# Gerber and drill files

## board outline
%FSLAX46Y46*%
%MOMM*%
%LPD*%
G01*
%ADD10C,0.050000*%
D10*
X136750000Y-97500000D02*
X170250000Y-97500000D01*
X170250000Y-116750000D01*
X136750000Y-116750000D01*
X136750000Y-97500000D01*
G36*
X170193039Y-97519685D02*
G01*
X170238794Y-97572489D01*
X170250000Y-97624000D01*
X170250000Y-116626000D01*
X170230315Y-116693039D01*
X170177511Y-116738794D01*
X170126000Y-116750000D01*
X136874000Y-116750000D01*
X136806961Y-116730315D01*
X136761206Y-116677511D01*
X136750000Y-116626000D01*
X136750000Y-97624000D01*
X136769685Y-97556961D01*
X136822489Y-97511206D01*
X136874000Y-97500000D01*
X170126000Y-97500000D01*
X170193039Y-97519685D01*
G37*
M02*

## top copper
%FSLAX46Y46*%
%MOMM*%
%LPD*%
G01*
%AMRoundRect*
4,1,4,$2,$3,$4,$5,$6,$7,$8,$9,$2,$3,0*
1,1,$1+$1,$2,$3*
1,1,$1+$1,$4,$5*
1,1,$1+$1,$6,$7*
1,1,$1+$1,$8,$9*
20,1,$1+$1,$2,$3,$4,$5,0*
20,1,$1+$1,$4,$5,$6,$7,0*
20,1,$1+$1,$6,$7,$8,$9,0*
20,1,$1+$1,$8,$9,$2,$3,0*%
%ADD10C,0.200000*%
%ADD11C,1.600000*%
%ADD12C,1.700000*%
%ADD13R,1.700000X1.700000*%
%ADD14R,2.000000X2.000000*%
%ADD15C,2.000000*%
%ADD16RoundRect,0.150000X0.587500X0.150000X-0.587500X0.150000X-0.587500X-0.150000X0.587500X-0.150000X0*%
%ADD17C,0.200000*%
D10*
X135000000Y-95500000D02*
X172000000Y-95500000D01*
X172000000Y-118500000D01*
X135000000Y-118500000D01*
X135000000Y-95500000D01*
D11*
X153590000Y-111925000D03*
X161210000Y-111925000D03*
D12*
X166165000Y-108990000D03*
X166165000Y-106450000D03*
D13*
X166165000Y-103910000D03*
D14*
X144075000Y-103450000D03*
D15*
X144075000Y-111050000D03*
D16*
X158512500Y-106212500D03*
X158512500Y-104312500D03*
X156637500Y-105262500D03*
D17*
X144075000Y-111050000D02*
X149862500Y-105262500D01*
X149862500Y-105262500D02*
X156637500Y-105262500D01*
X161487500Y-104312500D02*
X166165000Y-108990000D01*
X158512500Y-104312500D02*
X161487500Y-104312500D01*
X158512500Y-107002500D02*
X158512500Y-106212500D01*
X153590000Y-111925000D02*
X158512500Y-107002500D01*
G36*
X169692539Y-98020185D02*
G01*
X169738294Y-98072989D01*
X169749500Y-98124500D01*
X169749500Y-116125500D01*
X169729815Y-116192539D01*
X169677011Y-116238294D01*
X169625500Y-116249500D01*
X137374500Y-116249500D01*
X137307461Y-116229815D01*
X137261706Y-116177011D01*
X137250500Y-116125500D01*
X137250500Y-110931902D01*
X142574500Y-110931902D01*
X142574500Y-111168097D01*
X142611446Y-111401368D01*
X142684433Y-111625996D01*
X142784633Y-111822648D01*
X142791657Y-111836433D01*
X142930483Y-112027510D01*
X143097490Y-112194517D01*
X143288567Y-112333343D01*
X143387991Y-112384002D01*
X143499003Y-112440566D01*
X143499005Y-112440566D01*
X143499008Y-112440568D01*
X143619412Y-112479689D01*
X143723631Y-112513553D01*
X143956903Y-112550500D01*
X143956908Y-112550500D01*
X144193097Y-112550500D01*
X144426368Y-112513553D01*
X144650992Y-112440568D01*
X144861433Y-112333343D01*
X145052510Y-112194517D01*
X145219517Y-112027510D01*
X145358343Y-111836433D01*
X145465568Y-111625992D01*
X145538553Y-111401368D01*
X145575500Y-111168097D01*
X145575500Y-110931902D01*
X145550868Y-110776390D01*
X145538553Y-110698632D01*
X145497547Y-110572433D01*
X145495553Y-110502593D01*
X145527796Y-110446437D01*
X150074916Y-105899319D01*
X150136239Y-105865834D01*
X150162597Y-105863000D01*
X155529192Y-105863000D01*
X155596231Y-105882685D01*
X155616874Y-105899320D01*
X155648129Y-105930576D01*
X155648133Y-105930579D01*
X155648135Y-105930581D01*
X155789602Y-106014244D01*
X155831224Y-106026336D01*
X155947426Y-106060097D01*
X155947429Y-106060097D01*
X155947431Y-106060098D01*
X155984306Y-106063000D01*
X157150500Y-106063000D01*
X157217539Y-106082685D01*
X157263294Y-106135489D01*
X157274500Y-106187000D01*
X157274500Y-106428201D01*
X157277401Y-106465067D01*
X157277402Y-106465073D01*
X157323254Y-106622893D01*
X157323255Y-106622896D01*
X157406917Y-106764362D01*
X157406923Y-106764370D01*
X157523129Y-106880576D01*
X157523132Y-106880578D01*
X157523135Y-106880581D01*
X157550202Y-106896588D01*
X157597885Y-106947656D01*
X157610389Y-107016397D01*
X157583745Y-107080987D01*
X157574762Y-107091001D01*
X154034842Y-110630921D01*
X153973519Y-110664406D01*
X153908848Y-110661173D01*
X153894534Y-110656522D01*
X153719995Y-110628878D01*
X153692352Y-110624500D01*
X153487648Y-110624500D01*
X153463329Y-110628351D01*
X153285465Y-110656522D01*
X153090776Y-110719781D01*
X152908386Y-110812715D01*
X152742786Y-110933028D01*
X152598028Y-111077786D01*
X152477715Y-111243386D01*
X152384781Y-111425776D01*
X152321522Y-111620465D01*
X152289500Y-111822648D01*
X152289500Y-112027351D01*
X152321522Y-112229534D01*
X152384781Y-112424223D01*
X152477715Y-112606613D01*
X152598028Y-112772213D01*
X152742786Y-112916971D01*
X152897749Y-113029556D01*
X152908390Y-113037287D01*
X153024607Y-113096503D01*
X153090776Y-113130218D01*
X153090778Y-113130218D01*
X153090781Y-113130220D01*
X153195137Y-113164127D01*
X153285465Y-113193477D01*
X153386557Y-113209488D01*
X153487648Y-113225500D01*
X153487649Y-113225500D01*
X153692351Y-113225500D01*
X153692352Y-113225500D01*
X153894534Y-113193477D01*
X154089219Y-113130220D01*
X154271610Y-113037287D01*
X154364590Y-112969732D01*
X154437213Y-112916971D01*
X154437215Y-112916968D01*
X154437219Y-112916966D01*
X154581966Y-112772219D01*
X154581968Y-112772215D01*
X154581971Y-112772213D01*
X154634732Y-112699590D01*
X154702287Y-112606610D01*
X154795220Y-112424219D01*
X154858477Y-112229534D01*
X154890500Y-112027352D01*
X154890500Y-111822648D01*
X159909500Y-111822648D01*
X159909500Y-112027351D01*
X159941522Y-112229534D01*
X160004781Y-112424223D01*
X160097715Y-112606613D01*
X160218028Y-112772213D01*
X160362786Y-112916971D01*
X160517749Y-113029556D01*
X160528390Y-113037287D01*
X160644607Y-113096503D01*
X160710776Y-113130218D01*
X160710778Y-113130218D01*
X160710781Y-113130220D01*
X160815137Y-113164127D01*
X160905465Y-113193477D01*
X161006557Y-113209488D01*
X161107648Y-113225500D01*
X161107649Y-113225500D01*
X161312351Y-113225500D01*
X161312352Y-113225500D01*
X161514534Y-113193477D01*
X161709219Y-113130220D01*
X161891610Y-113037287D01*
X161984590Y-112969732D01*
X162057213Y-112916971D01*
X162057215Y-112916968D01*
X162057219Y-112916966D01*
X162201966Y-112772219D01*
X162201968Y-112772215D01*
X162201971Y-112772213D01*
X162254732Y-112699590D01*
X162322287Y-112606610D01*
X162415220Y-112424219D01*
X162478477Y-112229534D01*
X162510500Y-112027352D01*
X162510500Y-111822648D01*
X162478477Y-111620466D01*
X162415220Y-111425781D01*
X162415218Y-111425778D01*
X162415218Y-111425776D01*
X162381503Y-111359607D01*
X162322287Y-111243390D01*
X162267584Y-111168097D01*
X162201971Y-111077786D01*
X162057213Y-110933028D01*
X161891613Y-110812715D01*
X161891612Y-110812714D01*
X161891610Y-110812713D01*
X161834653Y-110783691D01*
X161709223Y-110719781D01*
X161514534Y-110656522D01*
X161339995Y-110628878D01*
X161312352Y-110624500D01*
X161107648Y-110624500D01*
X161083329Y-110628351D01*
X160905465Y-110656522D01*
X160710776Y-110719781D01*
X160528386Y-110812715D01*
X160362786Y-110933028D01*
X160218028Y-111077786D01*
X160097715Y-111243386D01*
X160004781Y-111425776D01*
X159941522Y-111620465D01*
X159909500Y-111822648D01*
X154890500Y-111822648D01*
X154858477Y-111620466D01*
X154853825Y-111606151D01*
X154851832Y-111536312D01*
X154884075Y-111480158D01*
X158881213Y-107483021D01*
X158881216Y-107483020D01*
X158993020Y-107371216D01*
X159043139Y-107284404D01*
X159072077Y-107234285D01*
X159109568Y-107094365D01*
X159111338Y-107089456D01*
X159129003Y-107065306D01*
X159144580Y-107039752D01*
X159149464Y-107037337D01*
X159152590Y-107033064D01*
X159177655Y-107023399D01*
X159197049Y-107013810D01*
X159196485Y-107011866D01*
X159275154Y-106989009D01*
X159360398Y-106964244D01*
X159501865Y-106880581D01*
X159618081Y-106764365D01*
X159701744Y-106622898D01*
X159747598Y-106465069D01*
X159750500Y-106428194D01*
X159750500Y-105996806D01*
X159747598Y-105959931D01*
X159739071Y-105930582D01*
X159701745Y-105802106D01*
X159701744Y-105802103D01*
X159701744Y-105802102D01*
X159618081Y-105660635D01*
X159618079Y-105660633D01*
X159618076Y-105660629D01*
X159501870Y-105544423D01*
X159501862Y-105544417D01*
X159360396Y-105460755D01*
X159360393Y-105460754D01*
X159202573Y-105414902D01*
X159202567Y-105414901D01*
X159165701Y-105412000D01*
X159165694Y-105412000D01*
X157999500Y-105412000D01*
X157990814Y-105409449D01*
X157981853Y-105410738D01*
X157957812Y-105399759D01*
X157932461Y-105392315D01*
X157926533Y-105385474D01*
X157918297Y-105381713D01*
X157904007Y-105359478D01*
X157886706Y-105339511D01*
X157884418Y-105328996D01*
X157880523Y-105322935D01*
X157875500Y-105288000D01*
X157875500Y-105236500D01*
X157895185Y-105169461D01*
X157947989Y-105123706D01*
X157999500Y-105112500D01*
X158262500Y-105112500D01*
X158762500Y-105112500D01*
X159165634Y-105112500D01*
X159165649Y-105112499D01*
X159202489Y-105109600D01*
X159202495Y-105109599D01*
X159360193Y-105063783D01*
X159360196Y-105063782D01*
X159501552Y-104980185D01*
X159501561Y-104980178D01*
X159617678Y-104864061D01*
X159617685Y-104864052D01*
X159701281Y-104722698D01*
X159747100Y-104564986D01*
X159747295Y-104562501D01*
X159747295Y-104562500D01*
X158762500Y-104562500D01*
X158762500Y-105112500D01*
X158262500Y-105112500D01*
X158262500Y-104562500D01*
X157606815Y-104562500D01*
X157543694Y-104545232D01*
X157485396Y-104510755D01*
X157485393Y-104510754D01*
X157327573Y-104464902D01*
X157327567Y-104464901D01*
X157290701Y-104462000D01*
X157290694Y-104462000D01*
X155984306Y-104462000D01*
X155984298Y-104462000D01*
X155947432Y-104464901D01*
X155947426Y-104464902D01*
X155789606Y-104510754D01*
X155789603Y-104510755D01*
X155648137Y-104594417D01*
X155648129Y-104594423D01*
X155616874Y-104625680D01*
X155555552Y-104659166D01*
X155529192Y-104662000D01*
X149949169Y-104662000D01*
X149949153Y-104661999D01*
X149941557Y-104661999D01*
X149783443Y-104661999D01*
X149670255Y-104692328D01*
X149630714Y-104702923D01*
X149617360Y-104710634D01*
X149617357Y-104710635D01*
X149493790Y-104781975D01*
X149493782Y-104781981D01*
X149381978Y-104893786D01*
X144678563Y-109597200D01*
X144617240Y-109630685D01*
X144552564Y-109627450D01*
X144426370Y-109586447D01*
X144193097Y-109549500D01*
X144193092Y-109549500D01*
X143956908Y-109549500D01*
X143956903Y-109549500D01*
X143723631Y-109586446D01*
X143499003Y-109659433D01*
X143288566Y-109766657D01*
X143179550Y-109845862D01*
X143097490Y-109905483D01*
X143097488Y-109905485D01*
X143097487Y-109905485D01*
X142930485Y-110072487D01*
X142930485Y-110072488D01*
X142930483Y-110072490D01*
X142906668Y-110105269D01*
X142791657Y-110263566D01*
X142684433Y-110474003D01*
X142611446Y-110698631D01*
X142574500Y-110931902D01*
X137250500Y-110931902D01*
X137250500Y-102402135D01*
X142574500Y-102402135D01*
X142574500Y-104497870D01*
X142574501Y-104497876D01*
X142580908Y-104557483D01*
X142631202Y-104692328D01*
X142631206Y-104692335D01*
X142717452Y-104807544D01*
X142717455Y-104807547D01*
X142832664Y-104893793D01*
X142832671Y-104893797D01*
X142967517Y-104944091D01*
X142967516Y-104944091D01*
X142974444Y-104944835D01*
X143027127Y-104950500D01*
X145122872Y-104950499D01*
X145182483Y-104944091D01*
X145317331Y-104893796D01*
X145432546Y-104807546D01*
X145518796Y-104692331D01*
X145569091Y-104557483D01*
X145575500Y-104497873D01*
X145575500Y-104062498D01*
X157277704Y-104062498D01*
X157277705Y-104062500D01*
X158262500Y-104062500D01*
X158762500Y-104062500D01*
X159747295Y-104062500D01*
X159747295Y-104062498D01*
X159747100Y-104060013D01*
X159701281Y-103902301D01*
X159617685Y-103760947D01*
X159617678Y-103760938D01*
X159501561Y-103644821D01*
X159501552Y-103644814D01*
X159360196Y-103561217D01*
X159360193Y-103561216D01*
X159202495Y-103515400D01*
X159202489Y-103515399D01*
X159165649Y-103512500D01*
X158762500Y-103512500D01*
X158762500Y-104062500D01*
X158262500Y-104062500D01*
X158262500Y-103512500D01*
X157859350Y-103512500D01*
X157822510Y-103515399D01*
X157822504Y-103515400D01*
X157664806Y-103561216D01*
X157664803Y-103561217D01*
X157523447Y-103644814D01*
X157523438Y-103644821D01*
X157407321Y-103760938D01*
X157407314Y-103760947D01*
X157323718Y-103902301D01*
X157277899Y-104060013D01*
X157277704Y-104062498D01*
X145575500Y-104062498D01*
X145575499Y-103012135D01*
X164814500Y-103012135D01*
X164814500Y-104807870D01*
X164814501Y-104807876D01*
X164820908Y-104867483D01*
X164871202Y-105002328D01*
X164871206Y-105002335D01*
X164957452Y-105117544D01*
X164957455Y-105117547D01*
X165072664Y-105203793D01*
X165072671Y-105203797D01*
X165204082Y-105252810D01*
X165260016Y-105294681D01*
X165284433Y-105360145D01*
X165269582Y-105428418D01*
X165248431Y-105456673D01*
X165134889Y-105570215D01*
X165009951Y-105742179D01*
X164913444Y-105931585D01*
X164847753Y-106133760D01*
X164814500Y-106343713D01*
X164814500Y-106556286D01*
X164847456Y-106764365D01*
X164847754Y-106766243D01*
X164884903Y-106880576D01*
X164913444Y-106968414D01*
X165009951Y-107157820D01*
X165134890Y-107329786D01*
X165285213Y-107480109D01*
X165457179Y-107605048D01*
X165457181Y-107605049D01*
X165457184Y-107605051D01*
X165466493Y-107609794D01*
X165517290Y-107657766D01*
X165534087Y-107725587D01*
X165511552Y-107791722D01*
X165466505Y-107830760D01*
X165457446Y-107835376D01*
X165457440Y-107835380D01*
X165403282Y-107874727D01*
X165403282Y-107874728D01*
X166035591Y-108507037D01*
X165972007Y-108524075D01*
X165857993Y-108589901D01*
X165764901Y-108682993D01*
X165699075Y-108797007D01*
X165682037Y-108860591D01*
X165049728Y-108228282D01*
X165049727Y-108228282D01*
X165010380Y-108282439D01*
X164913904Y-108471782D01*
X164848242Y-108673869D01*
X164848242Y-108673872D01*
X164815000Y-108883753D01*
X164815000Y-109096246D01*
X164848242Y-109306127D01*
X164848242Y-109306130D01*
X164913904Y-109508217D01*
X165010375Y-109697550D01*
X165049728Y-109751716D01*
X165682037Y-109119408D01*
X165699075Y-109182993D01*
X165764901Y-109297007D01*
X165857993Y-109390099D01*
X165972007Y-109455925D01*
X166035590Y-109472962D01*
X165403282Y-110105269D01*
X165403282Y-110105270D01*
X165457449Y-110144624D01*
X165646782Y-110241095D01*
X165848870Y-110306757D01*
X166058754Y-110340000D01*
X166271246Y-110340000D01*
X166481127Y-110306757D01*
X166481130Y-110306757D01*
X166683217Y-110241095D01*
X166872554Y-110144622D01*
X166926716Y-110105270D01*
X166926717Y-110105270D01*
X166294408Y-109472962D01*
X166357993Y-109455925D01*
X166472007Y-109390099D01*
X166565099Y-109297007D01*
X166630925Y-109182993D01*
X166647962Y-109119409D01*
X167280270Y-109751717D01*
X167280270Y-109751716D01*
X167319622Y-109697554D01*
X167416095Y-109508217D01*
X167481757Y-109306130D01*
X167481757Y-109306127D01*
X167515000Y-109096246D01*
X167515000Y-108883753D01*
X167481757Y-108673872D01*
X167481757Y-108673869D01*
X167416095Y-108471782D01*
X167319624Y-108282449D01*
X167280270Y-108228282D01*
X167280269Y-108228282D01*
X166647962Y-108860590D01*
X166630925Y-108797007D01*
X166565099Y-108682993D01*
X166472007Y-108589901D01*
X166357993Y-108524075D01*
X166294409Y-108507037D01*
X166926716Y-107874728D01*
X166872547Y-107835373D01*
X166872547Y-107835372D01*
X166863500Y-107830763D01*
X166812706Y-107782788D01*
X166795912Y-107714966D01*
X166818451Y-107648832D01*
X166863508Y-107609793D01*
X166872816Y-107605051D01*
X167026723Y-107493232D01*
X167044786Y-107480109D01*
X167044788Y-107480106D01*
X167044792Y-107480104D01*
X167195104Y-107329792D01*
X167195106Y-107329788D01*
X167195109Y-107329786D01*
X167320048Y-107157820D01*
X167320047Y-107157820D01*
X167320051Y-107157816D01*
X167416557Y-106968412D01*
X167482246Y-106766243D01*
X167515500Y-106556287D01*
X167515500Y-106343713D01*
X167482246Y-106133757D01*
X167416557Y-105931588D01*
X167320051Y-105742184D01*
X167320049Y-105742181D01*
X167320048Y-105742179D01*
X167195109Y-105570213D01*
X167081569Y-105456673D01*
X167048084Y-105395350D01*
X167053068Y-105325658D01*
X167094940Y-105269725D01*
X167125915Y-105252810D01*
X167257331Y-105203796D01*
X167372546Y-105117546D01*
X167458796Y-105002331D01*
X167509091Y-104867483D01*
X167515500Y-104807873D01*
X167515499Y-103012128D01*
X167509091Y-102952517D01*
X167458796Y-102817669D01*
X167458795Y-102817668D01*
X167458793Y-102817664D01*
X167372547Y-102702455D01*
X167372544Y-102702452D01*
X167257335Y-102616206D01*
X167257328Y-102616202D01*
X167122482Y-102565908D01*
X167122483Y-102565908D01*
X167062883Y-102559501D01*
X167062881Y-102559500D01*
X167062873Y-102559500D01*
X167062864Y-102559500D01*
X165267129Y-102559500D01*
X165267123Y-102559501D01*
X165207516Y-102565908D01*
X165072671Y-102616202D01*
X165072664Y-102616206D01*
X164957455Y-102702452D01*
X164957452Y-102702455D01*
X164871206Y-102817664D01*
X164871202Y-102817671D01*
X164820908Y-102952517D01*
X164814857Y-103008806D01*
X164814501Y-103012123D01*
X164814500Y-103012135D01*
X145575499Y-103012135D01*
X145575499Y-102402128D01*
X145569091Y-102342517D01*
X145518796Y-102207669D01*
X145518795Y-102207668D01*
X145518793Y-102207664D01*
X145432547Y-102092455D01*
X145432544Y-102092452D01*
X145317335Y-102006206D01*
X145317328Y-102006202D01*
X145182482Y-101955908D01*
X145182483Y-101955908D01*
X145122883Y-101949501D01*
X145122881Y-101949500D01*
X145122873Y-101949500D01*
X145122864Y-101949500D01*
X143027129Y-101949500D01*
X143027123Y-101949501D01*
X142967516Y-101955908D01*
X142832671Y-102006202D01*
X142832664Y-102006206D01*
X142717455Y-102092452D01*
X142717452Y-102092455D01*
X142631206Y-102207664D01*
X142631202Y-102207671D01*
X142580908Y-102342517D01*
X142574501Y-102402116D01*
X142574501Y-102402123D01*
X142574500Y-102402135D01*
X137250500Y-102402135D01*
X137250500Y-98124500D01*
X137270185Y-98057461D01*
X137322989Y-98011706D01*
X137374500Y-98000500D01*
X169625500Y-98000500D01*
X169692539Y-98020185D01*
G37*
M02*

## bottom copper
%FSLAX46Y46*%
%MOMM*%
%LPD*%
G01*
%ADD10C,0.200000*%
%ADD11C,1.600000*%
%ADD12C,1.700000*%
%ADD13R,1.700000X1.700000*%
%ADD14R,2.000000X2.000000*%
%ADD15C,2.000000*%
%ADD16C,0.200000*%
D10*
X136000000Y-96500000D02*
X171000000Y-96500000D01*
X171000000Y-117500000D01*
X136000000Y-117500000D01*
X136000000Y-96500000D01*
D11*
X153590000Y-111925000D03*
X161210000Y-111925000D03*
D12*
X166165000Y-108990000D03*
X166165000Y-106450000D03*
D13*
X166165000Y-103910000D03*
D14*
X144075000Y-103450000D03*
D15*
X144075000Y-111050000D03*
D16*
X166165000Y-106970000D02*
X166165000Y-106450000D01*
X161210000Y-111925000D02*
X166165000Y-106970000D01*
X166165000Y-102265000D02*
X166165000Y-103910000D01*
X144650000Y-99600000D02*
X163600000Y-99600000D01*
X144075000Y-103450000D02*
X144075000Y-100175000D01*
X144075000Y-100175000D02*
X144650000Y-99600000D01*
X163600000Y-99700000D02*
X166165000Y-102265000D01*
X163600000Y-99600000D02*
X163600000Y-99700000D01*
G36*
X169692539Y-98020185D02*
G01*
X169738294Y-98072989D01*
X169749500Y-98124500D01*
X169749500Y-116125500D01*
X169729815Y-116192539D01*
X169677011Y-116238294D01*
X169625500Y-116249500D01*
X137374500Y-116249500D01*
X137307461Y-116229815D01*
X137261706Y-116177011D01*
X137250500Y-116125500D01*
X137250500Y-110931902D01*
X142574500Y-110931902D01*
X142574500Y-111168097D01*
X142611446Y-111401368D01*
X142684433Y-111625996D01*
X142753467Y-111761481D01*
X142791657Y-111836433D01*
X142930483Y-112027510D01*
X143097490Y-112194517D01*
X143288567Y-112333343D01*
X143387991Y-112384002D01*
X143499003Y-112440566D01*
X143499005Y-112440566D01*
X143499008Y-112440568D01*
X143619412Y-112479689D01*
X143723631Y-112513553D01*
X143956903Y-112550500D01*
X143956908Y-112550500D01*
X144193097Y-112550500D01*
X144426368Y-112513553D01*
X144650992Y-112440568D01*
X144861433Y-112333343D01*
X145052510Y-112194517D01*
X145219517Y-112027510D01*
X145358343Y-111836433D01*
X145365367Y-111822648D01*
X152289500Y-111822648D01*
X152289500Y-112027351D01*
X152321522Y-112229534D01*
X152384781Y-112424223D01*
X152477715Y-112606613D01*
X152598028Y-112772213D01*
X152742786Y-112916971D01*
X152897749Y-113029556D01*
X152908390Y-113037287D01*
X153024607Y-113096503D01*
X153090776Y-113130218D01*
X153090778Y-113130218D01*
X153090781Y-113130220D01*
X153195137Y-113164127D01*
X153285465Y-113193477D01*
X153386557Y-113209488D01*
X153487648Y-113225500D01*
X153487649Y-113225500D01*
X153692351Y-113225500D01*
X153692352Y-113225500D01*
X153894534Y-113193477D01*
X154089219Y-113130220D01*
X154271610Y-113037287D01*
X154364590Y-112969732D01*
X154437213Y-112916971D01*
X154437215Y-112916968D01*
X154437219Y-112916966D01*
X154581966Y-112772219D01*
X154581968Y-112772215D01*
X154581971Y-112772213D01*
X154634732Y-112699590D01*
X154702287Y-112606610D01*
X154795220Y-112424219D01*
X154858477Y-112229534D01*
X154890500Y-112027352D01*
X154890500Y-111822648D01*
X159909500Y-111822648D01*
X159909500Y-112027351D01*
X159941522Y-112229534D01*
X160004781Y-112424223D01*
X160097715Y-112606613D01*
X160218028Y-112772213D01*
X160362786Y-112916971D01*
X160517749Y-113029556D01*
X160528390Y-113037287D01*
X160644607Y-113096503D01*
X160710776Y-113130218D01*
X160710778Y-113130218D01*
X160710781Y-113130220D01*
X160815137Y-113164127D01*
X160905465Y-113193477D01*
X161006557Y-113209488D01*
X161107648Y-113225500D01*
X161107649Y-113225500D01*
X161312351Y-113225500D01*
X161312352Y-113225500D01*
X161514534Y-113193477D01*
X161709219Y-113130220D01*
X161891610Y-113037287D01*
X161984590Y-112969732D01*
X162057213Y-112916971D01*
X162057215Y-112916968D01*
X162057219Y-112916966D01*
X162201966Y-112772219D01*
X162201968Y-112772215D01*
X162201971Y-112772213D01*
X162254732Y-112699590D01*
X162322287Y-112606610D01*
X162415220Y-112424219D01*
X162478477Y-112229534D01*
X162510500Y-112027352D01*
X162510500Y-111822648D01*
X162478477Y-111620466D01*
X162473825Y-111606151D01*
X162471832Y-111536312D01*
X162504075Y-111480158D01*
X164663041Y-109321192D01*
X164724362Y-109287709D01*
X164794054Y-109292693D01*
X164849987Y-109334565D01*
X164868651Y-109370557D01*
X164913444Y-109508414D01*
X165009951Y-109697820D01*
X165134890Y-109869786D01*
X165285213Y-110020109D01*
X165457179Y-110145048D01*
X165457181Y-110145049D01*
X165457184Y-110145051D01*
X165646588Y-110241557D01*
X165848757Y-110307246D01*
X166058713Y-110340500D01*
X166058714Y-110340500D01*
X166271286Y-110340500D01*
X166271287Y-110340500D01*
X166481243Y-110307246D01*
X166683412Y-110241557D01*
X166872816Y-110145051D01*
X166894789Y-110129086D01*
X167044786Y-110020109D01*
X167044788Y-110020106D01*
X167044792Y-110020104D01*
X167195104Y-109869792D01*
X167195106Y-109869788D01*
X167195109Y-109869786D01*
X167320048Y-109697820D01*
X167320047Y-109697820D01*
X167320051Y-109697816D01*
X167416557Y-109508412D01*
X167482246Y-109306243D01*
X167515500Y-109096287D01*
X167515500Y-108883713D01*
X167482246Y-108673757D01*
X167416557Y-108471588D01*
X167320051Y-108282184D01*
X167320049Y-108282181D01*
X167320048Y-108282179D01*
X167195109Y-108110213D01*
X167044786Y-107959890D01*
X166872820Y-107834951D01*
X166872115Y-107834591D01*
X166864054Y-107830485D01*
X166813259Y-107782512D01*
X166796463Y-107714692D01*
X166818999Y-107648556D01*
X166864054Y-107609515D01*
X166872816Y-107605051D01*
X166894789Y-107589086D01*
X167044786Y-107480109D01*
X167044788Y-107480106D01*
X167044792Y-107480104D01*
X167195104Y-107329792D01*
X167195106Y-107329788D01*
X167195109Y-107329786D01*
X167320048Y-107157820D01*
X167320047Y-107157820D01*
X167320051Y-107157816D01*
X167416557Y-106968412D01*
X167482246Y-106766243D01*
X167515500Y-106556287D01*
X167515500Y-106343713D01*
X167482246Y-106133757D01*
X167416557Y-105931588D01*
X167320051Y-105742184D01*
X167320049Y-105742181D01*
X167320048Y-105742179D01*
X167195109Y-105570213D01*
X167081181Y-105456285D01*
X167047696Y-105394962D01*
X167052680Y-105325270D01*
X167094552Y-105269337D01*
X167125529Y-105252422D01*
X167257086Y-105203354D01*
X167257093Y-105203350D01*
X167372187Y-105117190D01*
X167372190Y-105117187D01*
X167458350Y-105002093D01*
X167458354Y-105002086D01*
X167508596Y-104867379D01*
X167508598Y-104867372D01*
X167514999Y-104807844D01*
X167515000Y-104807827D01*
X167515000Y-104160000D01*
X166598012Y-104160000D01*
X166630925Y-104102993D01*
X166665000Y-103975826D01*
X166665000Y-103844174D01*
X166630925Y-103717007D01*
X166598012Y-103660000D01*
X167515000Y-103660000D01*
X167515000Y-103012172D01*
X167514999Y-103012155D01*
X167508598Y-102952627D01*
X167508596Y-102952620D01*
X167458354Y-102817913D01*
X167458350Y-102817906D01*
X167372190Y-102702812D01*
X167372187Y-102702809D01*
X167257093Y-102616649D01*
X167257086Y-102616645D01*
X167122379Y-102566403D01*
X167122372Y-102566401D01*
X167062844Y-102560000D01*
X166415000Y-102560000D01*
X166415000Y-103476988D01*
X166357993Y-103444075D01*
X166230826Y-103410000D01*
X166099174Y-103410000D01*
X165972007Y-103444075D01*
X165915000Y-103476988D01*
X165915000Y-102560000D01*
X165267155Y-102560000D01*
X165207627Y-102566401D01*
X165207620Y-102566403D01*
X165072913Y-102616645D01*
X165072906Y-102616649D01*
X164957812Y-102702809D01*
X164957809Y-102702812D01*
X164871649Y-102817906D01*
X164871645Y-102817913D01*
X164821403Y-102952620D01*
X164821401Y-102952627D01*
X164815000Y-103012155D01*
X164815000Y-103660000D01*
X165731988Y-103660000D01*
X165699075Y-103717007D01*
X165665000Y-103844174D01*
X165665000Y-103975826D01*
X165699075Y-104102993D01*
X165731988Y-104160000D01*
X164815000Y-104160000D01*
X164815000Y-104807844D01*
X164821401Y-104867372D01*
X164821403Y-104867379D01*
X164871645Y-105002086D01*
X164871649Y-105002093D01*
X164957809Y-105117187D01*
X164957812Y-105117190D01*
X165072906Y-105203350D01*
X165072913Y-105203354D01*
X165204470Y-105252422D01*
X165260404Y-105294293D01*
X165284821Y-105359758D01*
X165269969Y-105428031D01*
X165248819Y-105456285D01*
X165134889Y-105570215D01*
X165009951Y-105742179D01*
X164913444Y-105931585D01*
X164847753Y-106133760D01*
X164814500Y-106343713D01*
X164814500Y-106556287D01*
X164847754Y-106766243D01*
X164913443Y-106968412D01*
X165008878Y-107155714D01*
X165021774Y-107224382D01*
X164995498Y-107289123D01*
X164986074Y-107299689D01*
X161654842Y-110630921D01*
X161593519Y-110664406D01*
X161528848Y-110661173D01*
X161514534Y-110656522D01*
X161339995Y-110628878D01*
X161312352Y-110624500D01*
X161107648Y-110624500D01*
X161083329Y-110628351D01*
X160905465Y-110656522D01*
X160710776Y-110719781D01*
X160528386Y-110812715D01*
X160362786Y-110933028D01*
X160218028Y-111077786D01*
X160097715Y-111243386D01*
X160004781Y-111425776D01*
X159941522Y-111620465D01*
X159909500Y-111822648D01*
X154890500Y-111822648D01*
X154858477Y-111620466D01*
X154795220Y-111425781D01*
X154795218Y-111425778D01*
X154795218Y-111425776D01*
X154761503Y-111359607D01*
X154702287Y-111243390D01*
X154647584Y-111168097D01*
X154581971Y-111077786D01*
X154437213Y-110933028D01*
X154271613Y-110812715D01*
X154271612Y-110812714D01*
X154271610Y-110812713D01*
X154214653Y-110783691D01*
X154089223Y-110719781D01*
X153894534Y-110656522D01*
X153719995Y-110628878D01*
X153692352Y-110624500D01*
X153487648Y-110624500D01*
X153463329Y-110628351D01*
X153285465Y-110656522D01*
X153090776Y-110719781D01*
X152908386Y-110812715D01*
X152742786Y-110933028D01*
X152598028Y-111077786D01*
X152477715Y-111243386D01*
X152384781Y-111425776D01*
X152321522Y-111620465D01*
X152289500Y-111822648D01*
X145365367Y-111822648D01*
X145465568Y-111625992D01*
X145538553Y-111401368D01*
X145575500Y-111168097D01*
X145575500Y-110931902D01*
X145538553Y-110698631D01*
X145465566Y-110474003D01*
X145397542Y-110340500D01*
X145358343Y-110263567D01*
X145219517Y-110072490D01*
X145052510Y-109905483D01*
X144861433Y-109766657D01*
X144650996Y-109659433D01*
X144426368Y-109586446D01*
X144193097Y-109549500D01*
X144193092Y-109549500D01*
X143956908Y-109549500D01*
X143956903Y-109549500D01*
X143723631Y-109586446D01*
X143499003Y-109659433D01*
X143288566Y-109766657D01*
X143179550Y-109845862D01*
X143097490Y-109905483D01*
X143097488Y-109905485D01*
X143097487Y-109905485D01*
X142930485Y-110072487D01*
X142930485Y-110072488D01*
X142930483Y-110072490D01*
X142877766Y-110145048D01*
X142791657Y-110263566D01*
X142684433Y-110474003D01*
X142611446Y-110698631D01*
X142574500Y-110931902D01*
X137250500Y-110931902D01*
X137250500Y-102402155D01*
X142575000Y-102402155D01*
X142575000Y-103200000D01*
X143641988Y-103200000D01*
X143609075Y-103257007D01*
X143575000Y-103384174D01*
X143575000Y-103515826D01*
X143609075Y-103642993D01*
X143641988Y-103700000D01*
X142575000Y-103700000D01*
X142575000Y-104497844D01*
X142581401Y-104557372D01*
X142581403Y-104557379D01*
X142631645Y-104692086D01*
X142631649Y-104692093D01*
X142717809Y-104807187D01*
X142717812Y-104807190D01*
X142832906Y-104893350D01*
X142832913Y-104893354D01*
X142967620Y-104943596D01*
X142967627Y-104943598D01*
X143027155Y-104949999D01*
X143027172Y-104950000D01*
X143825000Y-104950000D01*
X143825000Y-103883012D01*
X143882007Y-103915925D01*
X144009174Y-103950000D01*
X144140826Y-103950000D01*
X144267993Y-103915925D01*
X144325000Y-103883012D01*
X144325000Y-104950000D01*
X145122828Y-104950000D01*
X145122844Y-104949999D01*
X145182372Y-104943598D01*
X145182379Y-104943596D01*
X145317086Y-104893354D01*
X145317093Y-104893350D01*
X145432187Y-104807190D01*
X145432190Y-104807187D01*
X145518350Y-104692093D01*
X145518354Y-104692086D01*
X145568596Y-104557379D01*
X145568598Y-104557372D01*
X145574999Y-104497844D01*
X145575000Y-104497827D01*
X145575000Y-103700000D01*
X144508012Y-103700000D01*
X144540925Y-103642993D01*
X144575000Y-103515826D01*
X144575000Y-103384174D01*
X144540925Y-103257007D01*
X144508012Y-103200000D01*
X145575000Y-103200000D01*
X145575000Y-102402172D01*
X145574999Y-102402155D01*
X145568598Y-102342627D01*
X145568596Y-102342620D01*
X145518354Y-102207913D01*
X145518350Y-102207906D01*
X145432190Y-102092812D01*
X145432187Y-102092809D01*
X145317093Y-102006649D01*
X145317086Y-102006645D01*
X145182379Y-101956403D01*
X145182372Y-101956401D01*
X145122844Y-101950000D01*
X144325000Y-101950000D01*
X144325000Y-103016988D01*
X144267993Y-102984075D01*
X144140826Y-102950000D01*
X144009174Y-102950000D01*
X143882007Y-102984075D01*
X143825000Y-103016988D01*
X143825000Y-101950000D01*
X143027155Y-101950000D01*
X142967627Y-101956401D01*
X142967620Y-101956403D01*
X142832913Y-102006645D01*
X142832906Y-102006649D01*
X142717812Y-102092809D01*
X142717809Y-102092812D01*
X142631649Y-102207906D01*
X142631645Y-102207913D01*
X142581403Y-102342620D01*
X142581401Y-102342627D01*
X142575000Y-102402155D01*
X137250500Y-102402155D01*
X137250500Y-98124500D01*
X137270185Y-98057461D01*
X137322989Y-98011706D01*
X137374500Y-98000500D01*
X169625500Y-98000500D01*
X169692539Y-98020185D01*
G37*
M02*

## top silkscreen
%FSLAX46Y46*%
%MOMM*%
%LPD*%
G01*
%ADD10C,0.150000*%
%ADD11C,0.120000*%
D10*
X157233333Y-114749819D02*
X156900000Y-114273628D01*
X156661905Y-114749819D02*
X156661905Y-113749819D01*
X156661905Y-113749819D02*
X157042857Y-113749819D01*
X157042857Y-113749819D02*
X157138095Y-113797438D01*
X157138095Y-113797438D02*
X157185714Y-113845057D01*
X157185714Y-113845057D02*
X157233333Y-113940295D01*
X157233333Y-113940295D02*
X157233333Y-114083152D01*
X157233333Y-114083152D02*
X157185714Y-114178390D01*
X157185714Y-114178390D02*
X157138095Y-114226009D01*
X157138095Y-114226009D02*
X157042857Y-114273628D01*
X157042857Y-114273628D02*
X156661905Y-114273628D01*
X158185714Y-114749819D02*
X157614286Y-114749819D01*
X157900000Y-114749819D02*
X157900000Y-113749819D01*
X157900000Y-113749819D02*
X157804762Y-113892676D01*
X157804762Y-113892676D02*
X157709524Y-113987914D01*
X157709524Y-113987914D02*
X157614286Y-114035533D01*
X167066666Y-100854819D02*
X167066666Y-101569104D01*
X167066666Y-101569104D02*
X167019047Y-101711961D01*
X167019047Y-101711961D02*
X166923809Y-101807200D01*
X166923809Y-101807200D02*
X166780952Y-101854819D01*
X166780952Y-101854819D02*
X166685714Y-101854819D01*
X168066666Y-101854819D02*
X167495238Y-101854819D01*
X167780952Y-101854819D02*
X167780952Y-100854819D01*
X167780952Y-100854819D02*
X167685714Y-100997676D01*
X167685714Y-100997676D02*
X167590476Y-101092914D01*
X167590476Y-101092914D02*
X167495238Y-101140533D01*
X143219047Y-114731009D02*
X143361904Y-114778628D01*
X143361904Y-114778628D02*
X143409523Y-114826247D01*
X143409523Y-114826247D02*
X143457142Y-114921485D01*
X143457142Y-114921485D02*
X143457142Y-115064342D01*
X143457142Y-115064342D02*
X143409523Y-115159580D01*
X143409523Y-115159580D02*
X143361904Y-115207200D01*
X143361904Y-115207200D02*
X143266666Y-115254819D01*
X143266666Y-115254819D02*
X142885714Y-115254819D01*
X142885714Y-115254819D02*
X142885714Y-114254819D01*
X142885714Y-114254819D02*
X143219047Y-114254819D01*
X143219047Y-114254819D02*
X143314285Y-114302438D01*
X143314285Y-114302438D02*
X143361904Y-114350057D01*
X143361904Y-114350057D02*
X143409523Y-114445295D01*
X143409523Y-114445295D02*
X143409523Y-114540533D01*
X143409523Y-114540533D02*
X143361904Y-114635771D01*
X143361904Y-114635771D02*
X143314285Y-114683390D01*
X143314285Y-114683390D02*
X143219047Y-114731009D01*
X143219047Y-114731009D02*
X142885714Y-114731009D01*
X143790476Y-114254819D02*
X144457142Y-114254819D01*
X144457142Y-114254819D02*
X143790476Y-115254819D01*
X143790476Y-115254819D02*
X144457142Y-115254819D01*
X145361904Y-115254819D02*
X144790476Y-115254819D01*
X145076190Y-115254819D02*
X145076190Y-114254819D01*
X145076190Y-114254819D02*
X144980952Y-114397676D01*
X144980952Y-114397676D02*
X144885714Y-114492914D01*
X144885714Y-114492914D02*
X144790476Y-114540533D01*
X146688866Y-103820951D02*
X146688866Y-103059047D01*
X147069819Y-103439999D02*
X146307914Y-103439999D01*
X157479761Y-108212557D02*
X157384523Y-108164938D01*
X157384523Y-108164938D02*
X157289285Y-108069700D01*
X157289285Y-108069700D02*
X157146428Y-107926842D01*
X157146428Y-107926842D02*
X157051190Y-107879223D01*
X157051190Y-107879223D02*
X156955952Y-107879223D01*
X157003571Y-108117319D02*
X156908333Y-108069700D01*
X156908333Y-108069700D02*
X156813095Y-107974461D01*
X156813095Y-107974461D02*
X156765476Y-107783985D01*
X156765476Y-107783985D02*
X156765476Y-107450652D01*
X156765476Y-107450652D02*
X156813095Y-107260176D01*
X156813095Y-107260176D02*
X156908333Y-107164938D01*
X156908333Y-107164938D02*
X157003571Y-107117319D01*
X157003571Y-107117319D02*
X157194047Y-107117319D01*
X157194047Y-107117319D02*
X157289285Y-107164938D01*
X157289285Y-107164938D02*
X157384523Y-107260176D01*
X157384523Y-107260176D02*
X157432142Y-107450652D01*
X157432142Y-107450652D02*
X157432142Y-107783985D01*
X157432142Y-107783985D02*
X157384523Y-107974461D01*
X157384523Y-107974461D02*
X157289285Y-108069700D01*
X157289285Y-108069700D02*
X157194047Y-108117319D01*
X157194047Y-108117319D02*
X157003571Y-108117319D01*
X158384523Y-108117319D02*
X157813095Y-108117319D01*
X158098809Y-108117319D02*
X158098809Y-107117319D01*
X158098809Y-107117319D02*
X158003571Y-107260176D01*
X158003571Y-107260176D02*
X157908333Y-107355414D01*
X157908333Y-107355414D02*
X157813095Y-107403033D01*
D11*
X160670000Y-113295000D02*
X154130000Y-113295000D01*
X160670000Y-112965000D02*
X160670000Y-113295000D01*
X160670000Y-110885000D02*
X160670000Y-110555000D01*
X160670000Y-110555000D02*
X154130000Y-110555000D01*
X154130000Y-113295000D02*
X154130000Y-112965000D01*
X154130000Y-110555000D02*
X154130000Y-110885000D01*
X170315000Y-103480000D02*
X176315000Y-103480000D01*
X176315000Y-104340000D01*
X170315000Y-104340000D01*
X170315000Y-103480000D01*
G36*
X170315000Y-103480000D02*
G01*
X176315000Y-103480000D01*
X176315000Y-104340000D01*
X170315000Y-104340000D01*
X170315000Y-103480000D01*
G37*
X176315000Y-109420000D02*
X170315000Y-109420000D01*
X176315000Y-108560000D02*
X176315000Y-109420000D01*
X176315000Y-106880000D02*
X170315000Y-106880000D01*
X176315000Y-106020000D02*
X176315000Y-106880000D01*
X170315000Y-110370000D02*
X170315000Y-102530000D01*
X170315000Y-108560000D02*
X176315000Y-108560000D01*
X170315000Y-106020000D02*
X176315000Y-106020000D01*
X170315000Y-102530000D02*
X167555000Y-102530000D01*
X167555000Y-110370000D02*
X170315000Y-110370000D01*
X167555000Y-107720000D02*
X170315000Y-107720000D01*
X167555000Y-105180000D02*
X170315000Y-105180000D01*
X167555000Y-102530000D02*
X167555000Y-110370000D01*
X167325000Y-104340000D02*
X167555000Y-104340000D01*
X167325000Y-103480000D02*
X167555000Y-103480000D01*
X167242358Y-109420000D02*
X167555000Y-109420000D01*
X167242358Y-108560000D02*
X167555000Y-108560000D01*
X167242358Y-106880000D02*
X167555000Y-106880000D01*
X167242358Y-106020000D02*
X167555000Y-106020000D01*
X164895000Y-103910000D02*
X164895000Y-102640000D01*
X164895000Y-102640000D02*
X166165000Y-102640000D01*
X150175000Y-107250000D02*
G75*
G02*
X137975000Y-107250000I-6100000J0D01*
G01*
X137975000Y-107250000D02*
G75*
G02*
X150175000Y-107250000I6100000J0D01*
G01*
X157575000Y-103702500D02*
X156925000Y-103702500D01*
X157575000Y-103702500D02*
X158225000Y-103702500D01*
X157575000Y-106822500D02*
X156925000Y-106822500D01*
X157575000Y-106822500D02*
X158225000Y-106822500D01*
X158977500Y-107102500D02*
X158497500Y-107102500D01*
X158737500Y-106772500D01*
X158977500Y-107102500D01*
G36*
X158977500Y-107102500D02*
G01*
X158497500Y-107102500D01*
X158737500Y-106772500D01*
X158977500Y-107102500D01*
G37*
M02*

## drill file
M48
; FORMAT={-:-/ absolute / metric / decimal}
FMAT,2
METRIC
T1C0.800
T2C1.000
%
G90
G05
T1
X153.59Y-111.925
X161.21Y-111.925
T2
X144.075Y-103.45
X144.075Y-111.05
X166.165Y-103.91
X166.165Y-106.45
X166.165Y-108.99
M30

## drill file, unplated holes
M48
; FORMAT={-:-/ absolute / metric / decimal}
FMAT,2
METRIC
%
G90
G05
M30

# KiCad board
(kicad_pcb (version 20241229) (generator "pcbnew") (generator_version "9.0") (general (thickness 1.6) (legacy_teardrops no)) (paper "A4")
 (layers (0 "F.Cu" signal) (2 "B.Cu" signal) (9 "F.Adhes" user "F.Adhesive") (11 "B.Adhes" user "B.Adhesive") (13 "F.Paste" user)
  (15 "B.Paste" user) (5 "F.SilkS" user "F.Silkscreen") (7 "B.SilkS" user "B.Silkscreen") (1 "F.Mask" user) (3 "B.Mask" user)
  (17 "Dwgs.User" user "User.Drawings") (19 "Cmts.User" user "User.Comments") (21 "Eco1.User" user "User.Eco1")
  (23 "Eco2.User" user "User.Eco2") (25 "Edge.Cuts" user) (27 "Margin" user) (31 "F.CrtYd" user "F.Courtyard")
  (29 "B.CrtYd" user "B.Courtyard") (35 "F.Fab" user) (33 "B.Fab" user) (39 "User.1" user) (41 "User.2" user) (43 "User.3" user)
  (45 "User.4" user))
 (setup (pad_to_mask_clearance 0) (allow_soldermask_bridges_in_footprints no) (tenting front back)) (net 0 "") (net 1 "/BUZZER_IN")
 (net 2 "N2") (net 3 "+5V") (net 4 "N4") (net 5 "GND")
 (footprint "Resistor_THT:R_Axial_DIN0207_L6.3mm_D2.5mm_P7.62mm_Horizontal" (layer "F.Cu") (at 161.21 111.925 180)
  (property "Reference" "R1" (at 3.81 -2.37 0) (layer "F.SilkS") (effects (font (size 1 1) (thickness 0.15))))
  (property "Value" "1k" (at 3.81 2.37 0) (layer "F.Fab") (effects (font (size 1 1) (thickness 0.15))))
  (fp_line (start 7.08 1.37) (end 7.08 1.04) (stroke (width 0.12) (type solid)) (layer "F.SilkS"))
  (fp_line (start 7.08 -1.37) (end 7.08 -1.04) (stroke (width 0.12) (type solid)) (layer "F.SilkS"))
  (fp_line (start 0.54 1.37) (end 7.08 1.37) (stroke (width 0.12) (type solid)) (layer "F.SilkS"))
  (fp_line (start 0.54 1.04) (end 0.54 1.37) (stroke (width 0.12) (type solid)) (layer "F.SilkS"))
  (fp_line (start 0.54 -1.04) (end 0.54 -1.37) (stroke (width 0.12) (type solid)) (layer "F.SilkS"))
  (fp_line (start 0.54 -1.37) (end 7.08 -1.37) (stroke (width 0.12) (type solid)) (layer "F.SilkS"))
  (pad "1" thru_hole circle (at 0 0 180) (size 1.6 1.6) (drill 0.8) (layers "*.Cu" "*.Mask") (remove_unused_layers no) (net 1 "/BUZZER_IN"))
  (pad "2" thru_hole circle (at 7.62 0 180) (size 1.6 1.6) (drill 0.8) (layers "*.Cu" "*.Mask") (remove_unused_layers no) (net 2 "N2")))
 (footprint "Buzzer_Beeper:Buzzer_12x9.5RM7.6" (layer "F.Cu") (at 144.075 103.45 -90)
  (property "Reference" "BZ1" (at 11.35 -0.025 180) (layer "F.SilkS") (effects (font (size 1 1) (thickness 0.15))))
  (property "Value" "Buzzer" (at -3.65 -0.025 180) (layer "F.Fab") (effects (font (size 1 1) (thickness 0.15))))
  (fp_circle (center 3.8 0) (end 9.9 0) (stroke (width 0.12) (type solid)) (fill no) (layer "F.SilkS"))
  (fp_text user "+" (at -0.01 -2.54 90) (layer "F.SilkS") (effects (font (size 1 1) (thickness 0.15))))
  (pad "1" thru_hole rect (at 0 0 270) (size 2 2) (drill 1) (layers "*.Cu" "*.Mask") (remove_unused_layers no) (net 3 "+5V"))
  (pad "2" thru_hole circle (at 7.6 0 270) (size 2 2) (drill 1) (layers "*.Cu" "*.Mask") (remove_unused_layers no) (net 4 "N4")))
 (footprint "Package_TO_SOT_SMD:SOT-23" (layer "F.Cu") (at 157.575 105.2625 180)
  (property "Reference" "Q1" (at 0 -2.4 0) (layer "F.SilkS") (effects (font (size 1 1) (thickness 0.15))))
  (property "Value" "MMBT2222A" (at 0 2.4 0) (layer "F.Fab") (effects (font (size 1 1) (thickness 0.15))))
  (fp_line (start 0 1.56) (end 0.65 1.56) (stroke (width 0.12) (type solid)) (layer "F.SilkS"))
  (fp_line (start 0 1.56) (end -0.65 1.56) (stroke (width 0.12) (type solid)) (layer "F.SilkS"))
  (fp_line (start 0 -1.56) (end 0.65 -1.56) (stroke (width 0.12) (type solid)) (layer "F.SilkS"))
  (fp_line (start 0 -1.56) (end -0.65 -1.56) (stroke (width 0.12) (type solid)) (layer "F.SilkS"))
  (fp_poly (pts (xy -1.1625 -1.51) (xy -1.4025 -1.84) (xy -0.9225 -1.84)) (stroke (width 0.12) (type solid)) (fill yes) (layer "F.SilkS"))
  (pad "1" smd roundrect (at -0.9375 -0.95 180) (size 1.475 0.6) (layers "F.Cu" "F.Mask" "F.Paste") (roundrect_rratio 0.25) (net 2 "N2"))
  (pad "2" smd roundrect (at -0.9375 0.95 180) (size 1.475 0.6) (layers "F.Cu" "F.Mask" "F.Paste") (roundrect_rratio 0.25) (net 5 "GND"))
  (pad "3" smd roundrect (at 0.9375 0 180) (size 1.475 0.6) (layers "F.Cu" "F.Mask" "F.Paste") (roundrect_rratio 0.25) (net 4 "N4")))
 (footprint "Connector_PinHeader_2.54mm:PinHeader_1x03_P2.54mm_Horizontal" (layer "F.Cu") (at 166.165 103.91)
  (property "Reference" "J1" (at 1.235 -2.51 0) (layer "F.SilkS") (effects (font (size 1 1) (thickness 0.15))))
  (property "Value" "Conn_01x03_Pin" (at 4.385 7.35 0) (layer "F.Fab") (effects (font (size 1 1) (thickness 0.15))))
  (fp_line (start -1.27 -1.27) (end 0 -1.27) (stroke (width 0.12) (type solid)) (layer "F.SilkS"))
  (fp_line (start -1.27 0) (end -1.27 -1.27) (stroke (width 0.12) (type solid)) (layer "F.SilkS"))
  (fp_line (start 1.077358 2.11) (end 1.39 2.11) (stroke (width 0.12) (type solid)) (layer "F.SilkS"))
  (fp_line (start 1.077358 2.97) (end 1.39 2.97) (stroke (width 0.12) (type solid)) (layer "F.SilkS"))
  (fp_line (start 1.077358 4.65) (end 1.39 4.65) (stroke (width 0.12) (type solid)) (layer "F.SilkS"))
  (fp_line (start 1.077358 5.51) (end 1.39 5.51) (stroke (width 0.12) (type solid)) (layer "F.SilkS"))
  (fp_line (start 1.16 -0.43) (end 1.39 -0.43) (stroke (width 0.12) (type solid)) (layer "F.SilkS"))
  (fp_line (start 1.16 0.43) (end 1.39 0.43) (stroke (width 0.12) (type solid)) (layer "F.SilkS"))
  (fp_line (start 1.39 -1.38) (end 1.39 6.46) (stroke (width 0.12) (type solid)) (layer "F.SilkS"))
  (fp_line (start 1.39 1.27) (end 4.15 1.27) (stroke (width 0.12) (type solid)) (layer "F.SilkS"))
  (fp_line (start 1.39 3.81) (end 4.15 3.81) (stroke (width 0.12) (type solid)) (layer "F.SilkS"))
  (fp_line (start 1.39 6.46) (end 4.15 6.46) (stroke (width 0.12) (type solid)) (layer "F.SilkS"))
  (fp_line (start 4.15 -1.38) (end 1.39 -1.38) (stroke (width 0.12) (type solid)) (layer "F.SilkS"))
  (fp_line (start 4.15 2.11) (end 10.15 2.11) (stroke (width 0.12) (type solid)) (layer "F.SilkS"))
  (fp_line (start 4.15 4.65) (end 10.15 4.65) (stroke (width 0.12) (type solid)) (layer "F.SilkS"))
  (fp_line (start 4.15 6.46) (end 4.15 -1.38) (stroke (width 0.12) (type solid)) (layer "F.SilkS"))
  (fp_line (start 10.15 2.11) (end 10.15 2.97) (stroke (width 0.12) (type solid)) (layer "F.SilkS"))
  (fp_line (start 10.15 2.97) (end 4.15 2.97) (stroke (width 0.12) (type solid)) (layer "F.SilkS"))
  (fp_line (start 10.15 4.65) (end 10.15 5.51) (stroke (width 0.12) (type solid)) (layer "F.SilkS"))
  (fp_line (start 10.15 5.51) (end 4.15 5.51) (stroke (width 0.12) (type solid)) (layer "F.SilkS"))
  (fp_rect (start 4.15 -0.43) (end 10.15 0.43) (stroke (width 0.12) (type solid)) (fill yes) (layer "F.SilkS"))
  (pad "1" thru_hole rect (at 0 0) (size 1.7 1.7) (drill 1) (layers "*.Cu" "*.Mask") (remove_unused_layers no) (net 3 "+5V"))
  (pad "2" thru_hole circle (at 0 2.54) (size 1.7 1.7) (drill 1) (layers "*.Cu" "*.Mask") (remove_unused_layers no) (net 1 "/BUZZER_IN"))
  (pad "3" thru_hole circle (at 0 5.08) (size 1.7 1.7) (drill 1) (layers "*.Cu" "*.Mask") (remove_unused_layers no) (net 5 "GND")))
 (gr_rect (start 135 95.5) (end 172 118.5) (stroke (width 0.2) (type default)) (fill no) (layer "F.Cu"))
 (gr_rect (start 136 96.5) (end 171 117.5) (stroke (width 0.2) (type default)) (fill no) (layer "B.Cu"))
 (gr_rect (start 136.75 97.5) (end 170.25 116.75) (stroke (width 0.05) (type default)) (fill no) (layer "Edge.Cuts"))
 (segment (start 166.165 102.265) (end 166.165 103.91) (width 0.2) (layer "B.Cu") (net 3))
 (segment (start 144.65 99.6) (end 163.6 99.6) (width 0.2) (layer "B.Cu") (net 3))
 (segment (start 144.075 103.45) (end 144.075 100.175) (width 0.2) (layer "B.Cu") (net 3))
 (segment (start 144.075 100.175) (end 144.65 99.6) (width 0.2) (layer "B.Cu") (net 3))
 (segment (start 163.6 99.7) (end 166.165 102.265) (width 0.2) (layer "B.Cu") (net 3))
 (segment (start 163.6 99.6) (end 163.6 99.7) (width 0.2) (layer "B.Cu") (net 3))
 (segment (start 144.075 111.05) (end 149.8625 105.2625) (width 0.2) (layer "F.Cu") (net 4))
 (segment (start 149.8625 105.2625) (end 156.6375 105.2625) (width 0.2) (layer "F.Cu") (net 4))
 (segment (start 161.4875 104.3125) (end 166.165 108.99) (width 0.2) (layer "F.Cu") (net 5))
 (segment (start 158.5125 104.3125) (end 161.4875 104.3125) (width 0.2) (layer "F.Cu") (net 5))
 (segment (start 161.21 111.925) (end 166.165 106.97) (width 0.2) (layer "B.Cu") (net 1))
 (segment (start 166.165 106.97) (end 166.165 106.45) (width 0.2) (layer "B.Cu") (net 1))
 (segment (start 158.5125 107.0025) (end 158.5125 106.2125) (width 0.2) (layer "F.Cu") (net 2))
 (segment (start 153.59 111.925) (end 158.5125 107.0025) (width 0.2) (layer "F.Cu") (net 2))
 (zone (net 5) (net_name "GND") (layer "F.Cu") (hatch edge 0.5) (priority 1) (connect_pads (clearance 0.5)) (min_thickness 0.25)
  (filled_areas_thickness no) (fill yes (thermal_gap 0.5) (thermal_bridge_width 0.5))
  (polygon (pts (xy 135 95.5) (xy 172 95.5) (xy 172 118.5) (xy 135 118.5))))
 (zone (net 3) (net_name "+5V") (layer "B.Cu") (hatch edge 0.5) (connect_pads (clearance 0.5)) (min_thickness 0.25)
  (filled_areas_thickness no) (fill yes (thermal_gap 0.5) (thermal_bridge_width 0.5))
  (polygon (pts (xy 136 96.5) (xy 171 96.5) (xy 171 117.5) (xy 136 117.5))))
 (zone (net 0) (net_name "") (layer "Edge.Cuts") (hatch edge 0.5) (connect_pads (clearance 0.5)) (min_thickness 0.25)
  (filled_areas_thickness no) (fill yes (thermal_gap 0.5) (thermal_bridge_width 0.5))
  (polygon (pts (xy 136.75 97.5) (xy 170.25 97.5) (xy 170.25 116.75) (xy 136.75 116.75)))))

